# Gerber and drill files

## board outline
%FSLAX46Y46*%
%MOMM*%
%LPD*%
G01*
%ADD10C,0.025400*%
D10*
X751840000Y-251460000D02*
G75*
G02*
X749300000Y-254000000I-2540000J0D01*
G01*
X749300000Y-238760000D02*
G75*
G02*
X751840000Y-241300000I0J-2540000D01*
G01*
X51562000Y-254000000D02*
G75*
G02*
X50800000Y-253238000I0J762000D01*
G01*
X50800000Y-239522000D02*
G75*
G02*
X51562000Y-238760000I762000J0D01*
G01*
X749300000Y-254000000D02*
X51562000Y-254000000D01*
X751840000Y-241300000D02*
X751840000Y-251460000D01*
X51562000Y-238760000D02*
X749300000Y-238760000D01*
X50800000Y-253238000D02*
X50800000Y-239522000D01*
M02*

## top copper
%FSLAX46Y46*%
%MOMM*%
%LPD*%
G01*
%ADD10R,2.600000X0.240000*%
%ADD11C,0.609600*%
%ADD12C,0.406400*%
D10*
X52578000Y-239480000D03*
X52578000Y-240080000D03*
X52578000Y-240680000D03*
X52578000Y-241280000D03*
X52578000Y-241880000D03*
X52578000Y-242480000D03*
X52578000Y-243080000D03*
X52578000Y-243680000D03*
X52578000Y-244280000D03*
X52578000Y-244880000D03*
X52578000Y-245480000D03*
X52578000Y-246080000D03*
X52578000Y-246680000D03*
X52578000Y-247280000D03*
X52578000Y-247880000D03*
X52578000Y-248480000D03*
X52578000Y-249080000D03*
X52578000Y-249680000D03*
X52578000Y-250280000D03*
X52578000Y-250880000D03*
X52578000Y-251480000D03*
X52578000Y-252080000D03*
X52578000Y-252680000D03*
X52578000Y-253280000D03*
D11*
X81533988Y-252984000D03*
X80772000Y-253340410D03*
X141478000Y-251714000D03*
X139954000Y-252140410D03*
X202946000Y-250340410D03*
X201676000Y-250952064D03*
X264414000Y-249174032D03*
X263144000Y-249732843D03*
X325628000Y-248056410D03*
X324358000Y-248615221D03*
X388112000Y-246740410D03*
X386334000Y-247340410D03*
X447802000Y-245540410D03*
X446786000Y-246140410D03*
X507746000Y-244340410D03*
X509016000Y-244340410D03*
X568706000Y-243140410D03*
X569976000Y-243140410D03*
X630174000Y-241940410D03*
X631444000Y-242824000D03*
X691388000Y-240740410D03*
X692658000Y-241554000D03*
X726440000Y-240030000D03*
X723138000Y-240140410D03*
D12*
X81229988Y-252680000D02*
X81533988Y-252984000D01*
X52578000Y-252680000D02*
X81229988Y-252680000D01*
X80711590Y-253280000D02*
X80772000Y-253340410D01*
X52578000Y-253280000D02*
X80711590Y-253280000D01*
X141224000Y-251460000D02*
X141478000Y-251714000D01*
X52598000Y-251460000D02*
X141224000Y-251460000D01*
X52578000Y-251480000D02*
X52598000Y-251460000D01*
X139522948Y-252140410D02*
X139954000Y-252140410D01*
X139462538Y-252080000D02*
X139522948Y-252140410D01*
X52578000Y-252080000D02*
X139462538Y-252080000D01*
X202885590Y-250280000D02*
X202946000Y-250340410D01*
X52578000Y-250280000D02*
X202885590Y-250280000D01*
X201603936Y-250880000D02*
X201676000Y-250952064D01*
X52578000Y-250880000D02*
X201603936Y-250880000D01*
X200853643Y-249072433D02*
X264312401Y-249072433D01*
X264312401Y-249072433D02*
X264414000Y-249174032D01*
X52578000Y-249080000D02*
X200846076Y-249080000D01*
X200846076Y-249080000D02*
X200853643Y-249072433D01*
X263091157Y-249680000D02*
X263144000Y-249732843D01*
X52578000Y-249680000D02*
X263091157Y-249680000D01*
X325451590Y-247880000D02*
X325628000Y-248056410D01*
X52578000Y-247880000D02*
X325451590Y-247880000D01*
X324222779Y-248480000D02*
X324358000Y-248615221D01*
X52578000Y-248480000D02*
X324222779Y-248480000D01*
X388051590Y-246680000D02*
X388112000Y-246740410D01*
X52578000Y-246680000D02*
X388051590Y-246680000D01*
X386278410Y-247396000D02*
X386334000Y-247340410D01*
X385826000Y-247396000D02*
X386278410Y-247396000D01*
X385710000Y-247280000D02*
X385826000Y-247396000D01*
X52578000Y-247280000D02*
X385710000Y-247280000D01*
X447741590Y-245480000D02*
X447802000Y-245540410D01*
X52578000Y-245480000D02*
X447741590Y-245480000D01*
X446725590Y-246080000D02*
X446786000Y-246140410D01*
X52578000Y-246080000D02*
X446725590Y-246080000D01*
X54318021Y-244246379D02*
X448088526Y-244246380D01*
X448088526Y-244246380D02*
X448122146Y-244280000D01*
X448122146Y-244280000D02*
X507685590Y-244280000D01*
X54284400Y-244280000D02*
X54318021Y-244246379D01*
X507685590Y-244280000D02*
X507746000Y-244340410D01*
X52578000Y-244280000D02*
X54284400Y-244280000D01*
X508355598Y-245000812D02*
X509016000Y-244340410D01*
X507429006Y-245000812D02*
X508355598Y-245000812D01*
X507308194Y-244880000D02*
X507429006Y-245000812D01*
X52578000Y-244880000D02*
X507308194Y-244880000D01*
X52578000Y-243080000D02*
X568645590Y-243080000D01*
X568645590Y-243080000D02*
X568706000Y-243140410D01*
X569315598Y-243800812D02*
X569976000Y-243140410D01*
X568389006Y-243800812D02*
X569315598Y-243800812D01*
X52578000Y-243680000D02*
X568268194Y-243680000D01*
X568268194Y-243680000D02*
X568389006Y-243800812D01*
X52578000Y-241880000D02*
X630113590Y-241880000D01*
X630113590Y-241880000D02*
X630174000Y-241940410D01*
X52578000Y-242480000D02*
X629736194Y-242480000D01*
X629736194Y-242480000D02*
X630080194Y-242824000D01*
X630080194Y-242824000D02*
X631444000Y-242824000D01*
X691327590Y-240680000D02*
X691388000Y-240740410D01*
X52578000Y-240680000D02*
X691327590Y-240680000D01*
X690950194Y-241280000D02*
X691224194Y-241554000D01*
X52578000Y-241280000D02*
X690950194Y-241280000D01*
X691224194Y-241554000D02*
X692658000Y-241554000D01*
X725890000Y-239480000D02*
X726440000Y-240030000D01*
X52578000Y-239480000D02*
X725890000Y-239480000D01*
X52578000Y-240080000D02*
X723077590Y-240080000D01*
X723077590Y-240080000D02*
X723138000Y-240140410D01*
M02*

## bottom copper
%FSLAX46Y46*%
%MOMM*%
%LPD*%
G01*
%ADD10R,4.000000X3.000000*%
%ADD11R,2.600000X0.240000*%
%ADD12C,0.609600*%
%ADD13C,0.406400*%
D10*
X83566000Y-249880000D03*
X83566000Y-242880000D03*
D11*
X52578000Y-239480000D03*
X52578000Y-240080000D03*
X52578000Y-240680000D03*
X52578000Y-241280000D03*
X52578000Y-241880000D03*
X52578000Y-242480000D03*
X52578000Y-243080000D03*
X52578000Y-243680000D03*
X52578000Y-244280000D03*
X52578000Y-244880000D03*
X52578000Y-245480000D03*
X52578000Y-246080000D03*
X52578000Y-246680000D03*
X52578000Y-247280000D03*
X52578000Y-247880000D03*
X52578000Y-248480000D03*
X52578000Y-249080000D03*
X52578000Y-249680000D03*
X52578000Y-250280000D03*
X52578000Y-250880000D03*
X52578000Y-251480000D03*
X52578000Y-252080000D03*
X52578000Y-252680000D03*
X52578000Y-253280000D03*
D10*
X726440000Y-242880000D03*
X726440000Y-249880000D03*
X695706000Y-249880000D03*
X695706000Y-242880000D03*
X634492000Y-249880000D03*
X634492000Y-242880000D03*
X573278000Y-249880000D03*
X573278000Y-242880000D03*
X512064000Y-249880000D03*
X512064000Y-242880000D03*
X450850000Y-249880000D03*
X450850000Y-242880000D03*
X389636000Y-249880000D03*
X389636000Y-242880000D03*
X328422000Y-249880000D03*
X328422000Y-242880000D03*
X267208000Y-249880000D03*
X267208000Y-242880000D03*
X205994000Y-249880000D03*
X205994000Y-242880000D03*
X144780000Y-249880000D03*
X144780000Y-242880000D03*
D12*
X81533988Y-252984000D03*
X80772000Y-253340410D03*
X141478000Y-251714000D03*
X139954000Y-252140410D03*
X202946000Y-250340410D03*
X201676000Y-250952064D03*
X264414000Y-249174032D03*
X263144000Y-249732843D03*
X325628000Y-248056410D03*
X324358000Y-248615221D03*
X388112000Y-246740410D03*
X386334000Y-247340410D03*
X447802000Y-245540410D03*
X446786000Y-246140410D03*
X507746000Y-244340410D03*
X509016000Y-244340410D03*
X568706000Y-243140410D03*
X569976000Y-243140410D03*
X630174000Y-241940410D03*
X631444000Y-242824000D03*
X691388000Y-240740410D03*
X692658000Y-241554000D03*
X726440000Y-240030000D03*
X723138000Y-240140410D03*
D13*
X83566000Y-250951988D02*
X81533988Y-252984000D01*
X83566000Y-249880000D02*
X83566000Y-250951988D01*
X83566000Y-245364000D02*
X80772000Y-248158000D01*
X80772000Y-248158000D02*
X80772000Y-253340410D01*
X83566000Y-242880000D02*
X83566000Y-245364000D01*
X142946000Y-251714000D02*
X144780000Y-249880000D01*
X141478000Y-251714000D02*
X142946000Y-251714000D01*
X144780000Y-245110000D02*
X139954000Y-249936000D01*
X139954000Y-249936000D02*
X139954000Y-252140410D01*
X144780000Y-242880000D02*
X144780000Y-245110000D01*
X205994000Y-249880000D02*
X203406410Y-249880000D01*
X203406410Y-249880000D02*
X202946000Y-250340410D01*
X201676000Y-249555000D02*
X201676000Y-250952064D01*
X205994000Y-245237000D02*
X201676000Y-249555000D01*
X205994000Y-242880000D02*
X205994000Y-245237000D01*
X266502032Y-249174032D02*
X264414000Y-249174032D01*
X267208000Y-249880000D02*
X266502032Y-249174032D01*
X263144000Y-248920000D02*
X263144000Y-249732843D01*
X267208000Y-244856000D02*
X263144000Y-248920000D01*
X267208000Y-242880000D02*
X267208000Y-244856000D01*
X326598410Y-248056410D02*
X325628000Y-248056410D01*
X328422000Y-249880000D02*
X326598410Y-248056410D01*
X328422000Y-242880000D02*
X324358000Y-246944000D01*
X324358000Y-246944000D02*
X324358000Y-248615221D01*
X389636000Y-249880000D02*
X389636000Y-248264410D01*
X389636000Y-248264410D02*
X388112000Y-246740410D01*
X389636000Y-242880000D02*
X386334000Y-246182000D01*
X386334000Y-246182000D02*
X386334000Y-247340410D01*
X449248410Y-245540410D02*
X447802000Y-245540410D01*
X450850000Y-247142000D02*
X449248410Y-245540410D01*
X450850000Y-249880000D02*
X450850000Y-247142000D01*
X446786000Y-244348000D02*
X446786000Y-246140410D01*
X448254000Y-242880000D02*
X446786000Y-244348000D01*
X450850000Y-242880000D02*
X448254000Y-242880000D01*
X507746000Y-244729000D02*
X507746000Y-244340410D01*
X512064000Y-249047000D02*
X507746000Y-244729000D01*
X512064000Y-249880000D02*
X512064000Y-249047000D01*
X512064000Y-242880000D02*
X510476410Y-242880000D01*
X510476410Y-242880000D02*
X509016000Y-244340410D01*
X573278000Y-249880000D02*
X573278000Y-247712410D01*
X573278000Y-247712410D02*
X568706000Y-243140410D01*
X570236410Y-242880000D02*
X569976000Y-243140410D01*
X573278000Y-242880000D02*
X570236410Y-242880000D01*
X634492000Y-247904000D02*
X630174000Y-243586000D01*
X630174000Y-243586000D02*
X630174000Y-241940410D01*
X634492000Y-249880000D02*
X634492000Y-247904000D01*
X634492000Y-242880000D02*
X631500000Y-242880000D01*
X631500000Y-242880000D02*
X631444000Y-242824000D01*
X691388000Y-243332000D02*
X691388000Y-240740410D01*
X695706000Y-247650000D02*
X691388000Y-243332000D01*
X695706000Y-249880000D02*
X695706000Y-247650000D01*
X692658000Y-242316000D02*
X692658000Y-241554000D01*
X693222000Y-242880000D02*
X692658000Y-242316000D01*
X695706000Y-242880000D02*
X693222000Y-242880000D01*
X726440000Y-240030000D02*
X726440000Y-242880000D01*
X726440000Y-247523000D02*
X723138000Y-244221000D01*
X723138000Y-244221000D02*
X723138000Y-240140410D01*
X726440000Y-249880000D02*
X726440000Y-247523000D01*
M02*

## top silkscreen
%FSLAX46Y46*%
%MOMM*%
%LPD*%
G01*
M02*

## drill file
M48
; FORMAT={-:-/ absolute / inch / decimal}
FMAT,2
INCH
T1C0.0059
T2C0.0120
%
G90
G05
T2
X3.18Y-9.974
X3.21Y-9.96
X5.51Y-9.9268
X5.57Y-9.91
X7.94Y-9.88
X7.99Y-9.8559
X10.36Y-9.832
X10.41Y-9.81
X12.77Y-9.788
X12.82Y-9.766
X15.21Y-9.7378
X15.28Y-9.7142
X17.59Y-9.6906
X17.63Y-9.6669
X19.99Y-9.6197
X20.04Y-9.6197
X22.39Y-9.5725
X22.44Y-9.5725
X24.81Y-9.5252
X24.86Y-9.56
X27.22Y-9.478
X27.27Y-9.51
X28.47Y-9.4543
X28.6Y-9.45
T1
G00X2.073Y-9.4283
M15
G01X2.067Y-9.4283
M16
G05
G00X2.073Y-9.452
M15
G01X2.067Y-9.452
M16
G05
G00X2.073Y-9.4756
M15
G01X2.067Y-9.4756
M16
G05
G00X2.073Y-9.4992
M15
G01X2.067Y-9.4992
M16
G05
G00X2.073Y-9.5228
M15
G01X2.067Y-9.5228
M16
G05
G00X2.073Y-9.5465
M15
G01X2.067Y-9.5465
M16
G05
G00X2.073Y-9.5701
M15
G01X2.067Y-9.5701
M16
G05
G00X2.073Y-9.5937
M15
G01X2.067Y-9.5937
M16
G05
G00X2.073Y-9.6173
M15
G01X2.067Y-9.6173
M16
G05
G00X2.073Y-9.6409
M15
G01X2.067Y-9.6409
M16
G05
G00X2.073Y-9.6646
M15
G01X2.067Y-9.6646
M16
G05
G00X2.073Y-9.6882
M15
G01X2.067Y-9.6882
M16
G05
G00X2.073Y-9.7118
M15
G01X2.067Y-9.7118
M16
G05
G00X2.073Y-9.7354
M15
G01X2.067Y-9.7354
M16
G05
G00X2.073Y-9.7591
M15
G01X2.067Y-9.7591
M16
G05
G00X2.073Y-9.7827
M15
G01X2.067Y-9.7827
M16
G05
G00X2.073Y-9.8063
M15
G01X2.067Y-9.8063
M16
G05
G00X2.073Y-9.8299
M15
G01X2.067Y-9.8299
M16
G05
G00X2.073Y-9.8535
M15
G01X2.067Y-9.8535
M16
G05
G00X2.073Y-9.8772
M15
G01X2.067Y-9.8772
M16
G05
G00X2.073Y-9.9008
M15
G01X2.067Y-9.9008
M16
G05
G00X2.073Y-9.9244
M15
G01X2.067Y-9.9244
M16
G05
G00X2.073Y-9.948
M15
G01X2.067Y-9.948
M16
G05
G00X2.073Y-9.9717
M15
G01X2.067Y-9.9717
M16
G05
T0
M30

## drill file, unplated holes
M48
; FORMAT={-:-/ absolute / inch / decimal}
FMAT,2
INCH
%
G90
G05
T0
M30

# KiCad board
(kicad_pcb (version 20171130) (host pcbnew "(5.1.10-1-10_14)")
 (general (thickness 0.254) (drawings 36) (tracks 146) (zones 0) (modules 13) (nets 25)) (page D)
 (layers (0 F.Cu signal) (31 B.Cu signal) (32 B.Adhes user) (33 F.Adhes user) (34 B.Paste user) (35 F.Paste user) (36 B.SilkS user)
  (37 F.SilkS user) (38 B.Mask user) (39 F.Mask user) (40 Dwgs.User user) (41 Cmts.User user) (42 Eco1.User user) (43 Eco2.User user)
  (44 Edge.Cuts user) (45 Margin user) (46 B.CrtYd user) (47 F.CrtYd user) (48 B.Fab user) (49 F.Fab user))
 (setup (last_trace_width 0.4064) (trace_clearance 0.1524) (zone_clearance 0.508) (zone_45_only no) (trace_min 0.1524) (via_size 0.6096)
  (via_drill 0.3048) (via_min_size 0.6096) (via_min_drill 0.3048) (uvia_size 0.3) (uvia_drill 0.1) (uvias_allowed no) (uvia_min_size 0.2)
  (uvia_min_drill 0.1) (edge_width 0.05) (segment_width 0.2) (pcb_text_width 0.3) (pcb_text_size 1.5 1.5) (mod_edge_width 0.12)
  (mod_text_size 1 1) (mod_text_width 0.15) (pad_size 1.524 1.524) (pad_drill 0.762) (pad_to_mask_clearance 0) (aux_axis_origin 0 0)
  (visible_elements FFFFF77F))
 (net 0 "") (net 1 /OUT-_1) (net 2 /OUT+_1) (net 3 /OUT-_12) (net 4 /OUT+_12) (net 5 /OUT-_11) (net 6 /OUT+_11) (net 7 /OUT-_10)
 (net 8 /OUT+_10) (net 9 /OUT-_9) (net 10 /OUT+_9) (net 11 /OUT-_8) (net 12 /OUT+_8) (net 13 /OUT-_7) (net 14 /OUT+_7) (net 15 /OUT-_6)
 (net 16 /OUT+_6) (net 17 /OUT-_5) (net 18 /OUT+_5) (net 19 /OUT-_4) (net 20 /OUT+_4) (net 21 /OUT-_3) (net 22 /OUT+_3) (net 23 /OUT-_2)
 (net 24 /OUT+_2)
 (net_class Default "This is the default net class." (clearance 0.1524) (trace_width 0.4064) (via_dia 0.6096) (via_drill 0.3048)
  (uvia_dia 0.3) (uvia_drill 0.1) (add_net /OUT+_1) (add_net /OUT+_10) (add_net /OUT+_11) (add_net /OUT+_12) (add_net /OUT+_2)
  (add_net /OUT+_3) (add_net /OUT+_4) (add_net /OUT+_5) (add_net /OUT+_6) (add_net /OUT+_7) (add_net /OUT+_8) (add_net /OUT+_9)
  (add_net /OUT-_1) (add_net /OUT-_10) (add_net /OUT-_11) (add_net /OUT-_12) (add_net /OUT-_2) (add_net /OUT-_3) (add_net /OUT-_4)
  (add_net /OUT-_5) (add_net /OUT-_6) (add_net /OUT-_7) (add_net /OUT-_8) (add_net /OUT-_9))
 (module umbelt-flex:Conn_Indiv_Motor (layer B.Cu) (at 83.566 246.38 90)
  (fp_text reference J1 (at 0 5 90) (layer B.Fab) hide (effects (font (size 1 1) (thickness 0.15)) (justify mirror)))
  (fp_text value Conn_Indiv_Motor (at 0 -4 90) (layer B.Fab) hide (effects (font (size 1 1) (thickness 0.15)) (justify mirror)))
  (pad 2 smd rect (at -3.5 0 90) (size 3 4) (layers B.Cu B.Mask) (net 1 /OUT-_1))
  (pad 1 smd rect (at 3.5 0 90) (size 3 4) (layers B.Cu B.Mask) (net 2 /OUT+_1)))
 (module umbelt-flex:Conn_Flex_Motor (layer F.Cu) (at 52.578 246.38 180)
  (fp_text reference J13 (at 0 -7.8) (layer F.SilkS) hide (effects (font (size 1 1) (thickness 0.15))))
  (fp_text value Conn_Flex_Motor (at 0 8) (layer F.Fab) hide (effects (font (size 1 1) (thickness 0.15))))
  (pad 24 thru_hole rect (at 0 6.9 180) (size 2.6 0.24) (drill oval 0.3 0.15) (layers *.Cu *.Mask) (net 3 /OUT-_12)
   (solder_paste_margin_ratio -0.2))
  (pad 23 thru_hole rect (at 0 6.3 180) (size 2.6 0.24) (drill oval 0.3 0.15) (layers *.Cu *.Mask) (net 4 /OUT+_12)
   (solder_paste_margin_ratio -0.2))
  (pad 22 thru_hole rect (at 0 5.7 180) (size 2.6 0.24) (drill oval 0.3 0.15) (layers *.Cu *.Mask) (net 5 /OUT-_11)
   (solder_paste_margin_ratio -0.2))
  (pad 21 thru_hole rect (at 0 5.1 180) (size 2.6 0.24) (drill oval 0.3 0.15) (layers *.Cu *.Mask) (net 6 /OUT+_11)
   (solder_paste_margin_ratio -0.2))
  (pad 20 thru_hole rect (at 0 4.5 180) (size 2.6 0.24) (drill oval 0.3 0.15) (layers *.Cu *.Mask) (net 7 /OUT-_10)
   (solder_paste_margin_ratio -0.2))
  (pad 19 thru_hole rect (at 0 3.9 180) (size 2.6 0.24) (drill oval 0.3 0.15) (layers *.Cu *.Mask) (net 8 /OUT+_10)
   (solder_paste_margin_ratio -0.2))
  (pad 18 thru_hole rect (at 0 3.3 180) (size 2.6 0.24) (drill oval 0.3 0.15) (layers *.Cu *.Mask) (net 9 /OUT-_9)
   (solder_paste_margin_ratio -0.2))
  (pad 17 thru_hole rect (at 0 2.7 180) (size 2.6 0.24) (drill oval 0.3 0.15) (layers *.Cu *.Mask) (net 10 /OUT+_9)
   (solder_paste_margin_ratio -0.2))
  (pad 16 thru_hole rect (at 0 2.1 180) (size 2.6 0.24) (drill oval 0.3 0.15) (layers *.Cu *.Mask) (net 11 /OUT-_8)
   (solder_paste_margin_ratio -0.2))
  (pad 15 thru_hole rect (at 0 1.5 180) (size 2.6 0.24) (drill oval 0.3 0.15) (layers *.Cu *.Mask) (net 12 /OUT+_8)
   (solder_paste_margin_ratio -0.2))
  (pad 14 thru_hole rect (at 0 0.9 180) (size 2.6 0.24) (drill oval 0.3 0.15) (layers *.Cu *.Mask) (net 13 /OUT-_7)
   (solder_paste_margin_ratio -0.2))
  (pad 13 thru_hole rect (at 0 0.3 180) (size 2.6 0.24) (drill oval 0.3 0.15) (layers *.Cu *.Mask) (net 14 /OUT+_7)
   (solder_paste_margin_ratio -0.2))
  (pad 12 thru_hole rect (at 0 -0.3 180) (size 2.6 0.24) (drill oval 0.3 0.15) (layers *.Cu *.Mask) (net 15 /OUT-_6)
   (solder_paste_margin_ratio -0.2))
  (pad 11 thru_hole rect (at 0 -0.9 180) (size 2.6 0.24) (drill oval 0.3 0.15) (layers *.Cu *.Mask) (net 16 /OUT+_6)
   (solder_paste_margin_ratio -0.2))
  (pad 10 thru_hole rect (at 0 -1.5 180) (size 2.6 0.24) (drill oval 0.3 0.15) (layers *.Cu *.Mask) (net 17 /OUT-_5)
   (solder_paste_margin_ratio -0.2))
  (pad 9 thru_hole rect (at 0 -2.1 180) (size 2.6 0.24) (drill oval 0.3 0.15) (layers *.Cu *.Mask) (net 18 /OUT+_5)
   (solder_paste_margin_ratio -0.2))
  (pad 8 thru_hole rect (at 0 -2.7 180) (size 2.6 0.24) (drill oval 0.3 0.15) (layers *.Cu *.Mask) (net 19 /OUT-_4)
   (solder_paste_margin_ratio -0.2))
  (pad 7 thru_hole rect (at 0 -3.3 180) (size 2.6 0.24) (drill oval 0.3 0.15) (layers *.Cu *.Mask) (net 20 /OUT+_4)
   (solder_paste_margin_ratio -0.2))
  (pad 6 thru_hole rect (at 0 -3.9 180) (size 2.6 0.24) (drill oval 0.3 0.15) (layers *.Cu *.Mask) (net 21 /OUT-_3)
   (solder_paste_margin_ratio -0.2))
  (pad 5 thru_hole rect (at 0 -4.5 180) (size 2.6 0.24) (drill oval 0.3 0.15) (layers *.Cu *.Mask) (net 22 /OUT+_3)
   (solder_paste_margin_ratio -0.2))
  (pad 4 thru_hole rect (at 0 -5.1 180) (size 2.6 0.24) (drill oval 0.3 0.15) (layers *.Cu *.Mask) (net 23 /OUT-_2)
   (solder_paste_margin_ratio -0.2))
  (pad 3 thru_hole rect (at 0 -5.7 180) (size 2.6 0.24) (drill oval 0.3 0.15) (layers *.Cu *.Mask) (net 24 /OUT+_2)
   (solder_paste_margin_ratio -0.2))
  (pad 2 thru_hole rect (at 0 -6.3 180) (size 2.6 0.24) (drill oval 0.3 0.15) (layers *.Cu *.Mask) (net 1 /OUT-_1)
   (solder_paste_margin_ratio -0.2))
  (pad 1 thru_hole rect (at 0 -6.9 180) (size 2.6 0.24) (drill oval 0.3 0.15) (layers *.Cu *.Mask) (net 2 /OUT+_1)
   (solder_paste_margin_ratio -0.2)))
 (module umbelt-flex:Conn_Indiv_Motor (layer B.Cu) (at 726.44 246.38 270)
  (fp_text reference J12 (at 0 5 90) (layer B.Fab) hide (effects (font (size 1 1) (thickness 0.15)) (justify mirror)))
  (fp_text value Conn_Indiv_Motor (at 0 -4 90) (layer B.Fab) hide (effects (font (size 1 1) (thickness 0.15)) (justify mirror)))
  (pad 2 smd rect (at -3.5 0 270) (size 3 4) (layers B.Cu B.Mask) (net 3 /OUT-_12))
  (pad 1 smd rect (at 3.5 0 270) (size 3 4) (layers B.Cu B.Mask) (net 4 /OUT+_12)))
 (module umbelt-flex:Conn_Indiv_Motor (layer B.Cu) (at 695.706 246.38 90)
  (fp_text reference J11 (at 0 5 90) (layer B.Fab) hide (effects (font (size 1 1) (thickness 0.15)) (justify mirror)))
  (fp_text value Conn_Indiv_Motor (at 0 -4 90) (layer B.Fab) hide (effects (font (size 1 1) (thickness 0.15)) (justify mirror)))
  (pad 2 smd rect (at -3.5 0 90) (size 3 4) (layers B.Cu B.Mask) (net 5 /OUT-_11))
  (pad 1 smd rect (at 3.5 0 90) (size 3 4) (layers B.Cu B.Mask) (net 6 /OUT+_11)))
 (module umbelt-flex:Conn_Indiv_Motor (layer B.Cu) (at 634.492 246.38 90)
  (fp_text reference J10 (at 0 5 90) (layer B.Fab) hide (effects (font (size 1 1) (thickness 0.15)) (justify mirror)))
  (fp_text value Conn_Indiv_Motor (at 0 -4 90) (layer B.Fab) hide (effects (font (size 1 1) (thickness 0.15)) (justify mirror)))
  (pad 2 smd rect (at -3.5 0 90) (size 3 4) (layers B.Cu B.Mask) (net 7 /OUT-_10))
  (pad 1 smd rect (at 3.5 0 90) (size 3 4) (layers B.Cu B.Mask) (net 8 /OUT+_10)))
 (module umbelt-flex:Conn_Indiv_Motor (layer B.Cu) (at 573.278 246.38 90)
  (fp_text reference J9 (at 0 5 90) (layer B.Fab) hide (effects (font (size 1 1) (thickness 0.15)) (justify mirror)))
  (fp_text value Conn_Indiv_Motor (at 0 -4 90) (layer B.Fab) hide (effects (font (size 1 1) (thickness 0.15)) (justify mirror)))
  (pad 2 smd rect (at -3.5 0 90) (size 3 4) (layers B.Cu B.Mask) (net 9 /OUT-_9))
  (pad 1 smd rect (at 3.5 0 90) (size 3 4) (layers B.Cu B.Mask) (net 10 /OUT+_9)))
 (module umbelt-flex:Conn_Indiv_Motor (layer B.Cu) (at 512.064 246.38 90)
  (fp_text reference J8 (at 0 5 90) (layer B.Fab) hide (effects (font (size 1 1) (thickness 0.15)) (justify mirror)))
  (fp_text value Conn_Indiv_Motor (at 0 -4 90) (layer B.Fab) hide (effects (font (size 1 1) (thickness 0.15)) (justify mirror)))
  (pad 2 smd rect (at -3.5 0 90) (size 3 4) (layers B.Cu B.Mask) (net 11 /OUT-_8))
  (pad 1 smd rect (at 3.5 0 90) (size 3 4) (layers B.Cu B.Mask) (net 12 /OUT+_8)))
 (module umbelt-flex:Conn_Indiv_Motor (layer B.Cu) (at 450.85 246.38 90)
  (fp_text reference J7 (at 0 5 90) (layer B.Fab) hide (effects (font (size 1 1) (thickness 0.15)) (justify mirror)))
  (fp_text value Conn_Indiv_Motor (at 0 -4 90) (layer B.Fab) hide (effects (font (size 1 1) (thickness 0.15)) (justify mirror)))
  (pad 2 smd rect (at -3.5 0 90) (size 3 4) (layers B.Cu B.Mask) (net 13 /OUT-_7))
  (pad 1 smd rect (at 3.5 0 90) (size 3 4) (layers B.Cu B.Mask) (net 14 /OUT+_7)))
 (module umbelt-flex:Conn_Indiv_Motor (layer B.Cu) (at 389.636 246.38 90)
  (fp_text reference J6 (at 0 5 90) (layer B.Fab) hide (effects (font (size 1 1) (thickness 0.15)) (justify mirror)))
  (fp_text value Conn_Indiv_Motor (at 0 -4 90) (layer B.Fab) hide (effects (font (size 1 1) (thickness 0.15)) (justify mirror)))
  (pad 2 smd rect (at -3.5 0 90) (size 3 4) (layers B.Cu B.Mask) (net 15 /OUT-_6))
  (pad 1 smd rect (at 3.5 0 90) (size 3 4) (layers B.Cu B.Mask) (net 16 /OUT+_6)))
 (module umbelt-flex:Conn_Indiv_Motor (layer B.Cu) (at 328.422 246.38 90)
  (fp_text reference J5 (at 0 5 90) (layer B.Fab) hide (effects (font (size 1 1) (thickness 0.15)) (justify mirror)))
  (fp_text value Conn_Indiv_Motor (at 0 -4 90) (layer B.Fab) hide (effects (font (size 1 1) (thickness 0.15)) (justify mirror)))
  (pad 2 smd rect (at -3.5 0 90) (size 3 4) (layers B.Cu B.Mask) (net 17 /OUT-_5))
  (pad 1 smd rect (at 3.5 0 90) (size 3 4) (layers B.Cu B.Mask) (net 18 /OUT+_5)))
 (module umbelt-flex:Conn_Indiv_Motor (layer B.Cu) (at 267.208 246.38 90)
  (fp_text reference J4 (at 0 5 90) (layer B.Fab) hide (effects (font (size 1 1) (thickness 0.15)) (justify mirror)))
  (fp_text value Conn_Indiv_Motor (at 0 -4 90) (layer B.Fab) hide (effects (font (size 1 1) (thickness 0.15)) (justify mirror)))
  (pad 2 smd rect (at -3.5 0 90) (size 3 4) (layers B.Cu B.Mask) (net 19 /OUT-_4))
  (pad 1 smd rect (at 3.5 0 90) (size 3 4) (layers B.Cu B.Mask) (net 20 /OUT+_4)))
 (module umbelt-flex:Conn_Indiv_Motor (layer B.Cu) (at 205.994 246.38 90)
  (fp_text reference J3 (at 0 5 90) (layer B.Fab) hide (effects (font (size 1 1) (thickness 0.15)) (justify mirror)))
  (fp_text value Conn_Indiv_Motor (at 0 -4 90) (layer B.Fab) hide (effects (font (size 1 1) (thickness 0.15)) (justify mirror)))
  (pad 2 smd rect (at -3.5 0 90) (size 3 4) (layers B.Cu B.Mask) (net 21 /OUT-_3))
  (pad 1 smd rect (at 3.5 0 90) (size 3 4) (layers B.Cu B.Mask) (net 22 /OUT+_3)))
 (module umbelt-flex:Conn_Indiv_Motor (layer B.Cu) (at 144.78 246.38 90)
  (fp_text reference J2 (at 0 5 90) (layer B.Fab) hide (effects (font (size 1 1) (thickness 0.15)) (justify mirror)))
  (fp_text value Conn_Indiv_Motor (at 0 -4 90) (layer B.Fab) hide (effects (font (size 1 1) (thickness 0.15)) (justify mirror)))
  (pad 2 smd rect (at -3.5 0 90) (size 3 4) (layers B.Cu B.Mask) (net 23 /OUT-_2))
  (pad 1 smd rect (at 3.5 0 90) (size 3 4) (layers B.Cu B.Mask) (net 24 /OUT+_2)))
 (gr_arc (start 749.3 251.46) (end 749.3 254) (angle -90) (layer Edge.Cuts) (width 0.0254))
 (gr_arc (start 749.3 241.3) (end 751.84 241.3) (angle -90) (layer Edge.Cuts) (width 0.0254))
 (gr_arc (start 51.562 253.238) (end 50.8 253.238) (angle -90) (layer Edge.Cuts) (width 0.0254))
 (gr_arc (start 51.562 239.522) (end 51.562 238.76) (angle -90) (layer Edge.Cuts) (width 0.0254))
 (gr_line (start 749.3 254) (end 51.562 254) (layer Edge.Cuts) (width 0.0254))
 (gr_line (start 751.84 241.3) (end 751.84 251.46) (layer Edge.Cuts) (width 0.0254))
 (gr_line (start 51.562 238.76) (end 749.3 238.76) (layer Edge.Cuts) (width 0.0254))
 (gr_line (start 50.8 253.238) (end 50.8 239.522) (layer Edge.Cuts) (width 0.0254))
 (segment (start 83.566 250.951988) (end 81.533988 252.984) (width 0.4064) (layer B.Cu) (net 1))
 (via (at 81.533988 252.984) (size 0.6096) (drill 0.3048) (layers F.Cu B.Cu) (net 1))
 (segment (start 83.566 249.88) (end 83.566 250.951988) (width 0.4064) (layer B.Cu) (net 1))
 (segment (start 81.229988 252.68) (end 81.533988 252.984) (width 0.4064) (layer F.Cu) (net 1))
 (segment (start 52.578 252.68) (end 81.229988 252.68) (width 0.4064) (layer F.Cu) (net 1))
 (via (at 80.772 253.34041) (size 0.6096) (drill 0.3048) (layers F.Cu B.Cu) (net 2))
 (segment (start 80.71159 253.28) (end 80.772 253.34041) (width 0.4064) (layer F.Cu) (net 2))
 (segment (start 52.578 253.28) (end 80.71159 253.28) (width 0.4064) (layer F.Cu) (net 2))
 (segment (start 83.566 245.364) (end 80.772 248.158) (width 0.4064) (layer B.Cu) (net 2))
 (segment (start 80.772 248.158) (end 80.772 253.34041) (width 0.4064) (layer B.Cu) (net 2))
 (segment (start 83.566 242.88) (end 83.566 245.364) (width 0.4064) (layer B.Cu) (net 2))
 (via (at 141.478 251.714) (size 0.6096) (drill 0.3048) (layers F.Cu B.Cu) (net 23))
 (segment (start 142.946 251.714) (end 144.78 249.88) (width 0.4064) (layer B.Cu) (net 23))
 (segment (start 141.478 251.714) (end 142.946 251.714) (width 0.4064) (layer B.Cu) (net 23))
 (segment (start 141.224 251.46) (end 141.478 251.714) (width 0.4064) (layer F.Cu) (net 23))
 (segment (start 52.598 251.46) (end 141.224 251.46) (width 0.4064) (layer F.Cu) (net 23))
 (segment (start 52.578 251.48) (end 52.598 251.46) (width 0.4064) (layer F.Cu) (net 23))
 (via (at 139.954 252.14041) (size 0.6096) (drill 0.3048) (layers F.Cu B.Cu) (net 24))
 (segment (start 139.522948 252.14041) (end 139.954 252.14041) (width 0.4064) (layer F.Cu) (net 24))
 (segment (start 139.462538 252.08) (end 139.522948 252.14041) (width 0.4064) (layer F.Cu) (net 24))
 (segment (start 52.578 252.08) (end 139.462538 252.08) (width 0.4064) (layer F.Cu) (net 24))
 (segment (start 144.78 245.11) (end 139.954 249.936) (width 0.4064) (layer B.Cu) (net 24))
 (segment (start 139.954 249.936) (end 139.954 252.14041) (width 0.4064) (layer B.Cu) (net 24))
 (segment (start 144.78 242.88) (end 144.78 245.11) (width 0.4064) (layer B.Cu) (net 24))
 (segment (start 202.88559 250.28) (end 202.946 250.34041) (width 0.4064) (layer F.Cu) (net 21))
 (via (at 202.946 250.34041) (size 0.6096) (drill 0.3048) (layers F.Cu B.Cu) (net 21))
 (segment (start 52.578 250.28) (end 202.88559 250.28) (width 0.4064) (layer F.Cu) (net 21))
 (segment (start 205.994 249.88) (end 203.40641 249.88) (width 0.4064) (layer B.Cu) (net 21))
 (segment (start 203.40641 249.88) (end 202.946 250.34041) (width 0.4064) (layer B.Cu) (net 21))
 (via (at 201.676 250.952064) (size 0.6096) (drill 0.3048) (layers F.Cu B.Cu) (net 22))
 (segment (start 201.603936 250.88) (end 201.676 250.952064) (width 0.4064) (layer F.Cu) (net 22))
 (segment (start 52.578 250.88) (end 201.603936 250.88) (width 0.4064) (layer F.Cu) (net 22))
 (segment (start 201.676 249.555) (end 201.676 250.952064) (width 0.4064) (layer B.Cu) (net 22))
 (segment (start 205.994 245.237) (end 201.676 249.555) (width 0.4064) (layer B.Cu) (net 22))
 (segment (start 205.994 242.88) (end 205.994 245.237) (width 0.4064) (layer B.Cu) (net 22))
 (segment (start 266.502032 249.174032) (end 264.414 249.174032) (width 0.4064) (layer B.Cu) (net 19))
 (via (at 264.414 249.174032) (size 0.6096) (drill 0.3048) (layers F.Cu B.Cu) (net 19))
 (segment (start 200.853643 249.072433) (end 264.312401 249.072433) (width 0.4064) (layer F.Cu) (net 19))
 (segment (start 264.312401 249.072433) (end 264.414 249.174032) (width 0.4064) (layer F.Cu) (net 19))
 (segment (start 52.578 249.08) (end 200.846076 249.08) (width 0.4064) (layer F.Cu) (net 19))
 (segment (start 200.846076 249.08) (end 200.853643 249.072433) (width 0.4064) (layer F.Cu) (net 19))
 (segment (start 267.208 249.88) (end 266.502032 249.174032) (width 0.4064) (layer B.Cu) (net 19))
 (via (at 263.144 249.732843) (size 0.6096) (drill 0.3048) (layers F.Cu B.Cu) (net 20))
 (segment (start 263.091157 249.68) (end 263.144 249.732843) (width 0.4064) (layer F.Cu) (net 20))
 (segment (start 52.578 249.68) (end 263.091157 249.68) (width 0.4064) (layer F.Cu) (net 20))
 (segment (start 263.144 248.92) (end 263.144 249.732843) (width 0.4064) (layer B.Cu) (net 20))
 (segment (start 267.208 244.856) (end 263.144 248.92) (width 0.4064) (layer B.Cu) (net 20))
 (segment (start 267.208 242.88) (end 267.208 244.856) (width 0.4064) (layer B.Cu) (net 20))
 (via (at 325.628 248.05641) (size 0.6096) (drill 0.3048) (layers F.Cu B.Cu) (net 17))
 (segment (start 326.59841 248.05641) (end 325.628 248.05641) (width 0.4064) (layer B.Cu) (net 17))
 (segment (start 328.422 249.88) (end 326.59841 248.05641) (width 0.4064) (layer B.Cu) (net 17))
 (segment (start 325.45159 247.88) (end 325.628 248.05641) (width 0.4064) (layer F.Cu) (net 17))
 (segment (start 52.578 247.88) (end 325.45159 247.88) (width 0.4064) (layer F.Cu) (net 17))
 (segment (start 328.422 242.88) (end 324.358 246.944) (width 0.4064) (layer B.Cu) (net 18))
 (via (at 324.358 248.615221) (size 0.6096) (drill 0.3048) (layers F.Cu B.Cu) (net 18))
 (segment (start 324.358 246.944) (end 324.358 248.615221) (width 0.4064) (layer B.Cu) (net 18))
 (segment (start 324.222779 248.48) (end 324.358 248.615221) (width 0.4064) (layer F.Cu) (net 18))
 (segment (start 52.578 248.48) (end 324.222779 248.48) (width 0.4064) (layer F.Cu) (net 18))
 (via (at 388.112 246.74041) (size 0.6096) (drill 0.3048) (layers F.Cu B.Cu) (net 15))
 (segment (start 389.636 249.88) (end 389.636 248.26441) (width 0.4064) (layer B.Cu) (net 15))
 (segment (start 389.636 248.26441) (end 388.112 246.74041) (width 0.4064) (layer B.Cu) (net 15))
 (segment (start 388.05159 246.68) (end 388.112 246.74041) (width 0.4064) (layer F.Cu) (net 15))
 (segment (start 52.578 246.68) (end 388.05159 246.68) (width 0.4064) (layer F.Cu) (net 15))
 (via (at 386.334 247.34041) (size 0.6096) (drill 0.3048) (layers F.Cu B.Cu) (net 16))
 (segment (start 389.636 242.88) (end 386.334 246.182) (width 0.4064) (layer B.Cu) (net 16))
 (segment (start 386.334 246.182) (end 386.334 247.34041) (width 0.4064) (layer B.Cu) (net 16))
 (segment (start 386.27841 247.396) (end 386.334 247.34041) (width 0.4064) (layer F.Cu) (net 16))
 (segment (start 385.826 247.396) (end 386.27841 247.396) (width 0.4064) (layer F.Cu) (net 16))
 (segment (start 385.71 247.28) (end 385.826 247.396) (width 0.4064) (layer F.Cu) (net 16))
 (segment (start 52.578 247.28) (end 385.71 247.28) (width 0.4064) (layer F.Cu) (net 16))
 (via (at 447.802 245.54041) (size 0.6096) (drill 0.3048) (layers F.Cu B.Cu) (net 13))
 (segment (start 447.74159 245.48) (end 447.802 245.54041) (width 0.4064) (layer F.Cu) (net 13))
 (segment (start 52.578 245.48) (end 447.74159 245.48) (width 0.4064) (layer F.Cu) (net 13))
 (segment (start 449.24841 245.54041) (end 447.802 245.54041) (width 0.4064) (layer B.Cu) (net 13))
 (segment (start 450.85 247.142) (end 449.24841 245.54041) (width 0.4064) (layer B.Cu) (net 13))
 (segment (start 450.85 249.88) (end 450.85 247.142) (width 0.4064) (layer B.Cu) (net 13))
 (via (at 446.786 246.14041) (size 0.6096) (drill 0.3048) (layers F.Cu B.Cu) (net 14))
 (segment (start 446.72559 246.08) (end 446.786 246.14041) (width 0.4064) (layer F.Cu) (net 14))
 (segment (start 52.578 246.08) (end 446.72559 246.08) (width 0.4064) (layer F.Cu) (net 14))
 (segment (start 446.786 244.348) (end 446.786 246.14041) (width 0.4064) (layer B.Cu) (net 14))
 (segment (start 448.254 242.88) (end 446.786 244.348) (width 0.4064) (layer B.Cu) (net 14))
 (segment (start 450.85 242.88) (end 448.254 242.88) (width 0.4064) (layer B.Cu) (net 14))
 (via (at 507.746 244.34041) (size 0.6096) (drill 0.3048) (layers F.Cu B.Cu) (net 11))
 (segment (start 54.318021 244.246379) (end 448.088526 244.24638) (width 0.4064) (layer F.Cu) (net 11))
 (segment (start 448.088526 244.24638) (end 448.122146 244.28) (width 0.4064) (layer F.Cu) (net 11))
 (segment (start 448.122146 244.28) (end 507.68559 244.28) (width 0.4064) (layer F.Cu) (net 11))
 (segment (start 54.2844 244.28) (end 54.318021 244.246379) (width 0.4064) (layer F.Cu) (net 11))
 (segment (start 507.68559 244.28) (end 507.746 244.34041) (width 0.4064) (layer F.Cu) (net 11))
 (segment (start 52.578 244.28) (end 54.2844 244.28) (width 0.4064) (layer F.Cu) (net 11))
 (segment (start 507.746 244.729) (end 507.746 244.34041) (width 0.4064) (layer B.Cu) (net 11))
 (segment (start 512.064 249.047) (end 507.746 244.729) (width 0.4064) (layer B.Cu) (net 11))
 (segment (start 512.064 249.88) (end 512.064 249.047) (width 0.4064) (layer B.Cu) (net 11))
 (via (at 509.016 244.34041) (size 0.6096) (drill 0.3048) (layers F.Cu B.Cu) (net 12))
 (segment (start 512.064 242.88) (end 510.47641 242.88) (width 0.4064) (layer B.Cu) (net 12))
 (segment (start 510.47641 242.88) (end 509.016 244.34041) (width 0.4064) (layer B.Cu) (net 12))
 (segment (start 508.355598 245.000812) (end 509.016 244.34041) (width 0.4064) (layer F.Cu) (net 12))
 (segment (start 507.429006 245.000812) (end 508.355598 245.000812) (width 0.4064) (layer F.Cu) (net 12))
 (segment (start 507.308194 244.88) (end 507.429006 245.000812) (width 0.4064) (layer F.Cu) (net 12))
 (segment (start 52.578 244.88) (end 507.308194 244.88) (width 0.4064) (layer F.Cu) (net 12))
 (via (at 568.706 243.14041) (size 0.6096) (drill 0.3048) (layers F.Cu B.Cu) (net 9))
 (segment (start 573.278 249.88) (end 573.278 247.71241) (width 0.4064) (layer B.Cu) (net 9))
 (segment (start 573.278 247.71241) (end 568.706 243.14041) (width 0.4064) (layer B.Cu) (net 9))
 (segment (start 52.578 243.08) (end 568.64559 243.08) (width 0.4064) (layer F.Cu) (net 9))
 (segment (start 568.64559 243.08) (end 568.706 243.14041) (width 0.4064) (layer F.Cu) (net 9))
 (via (at 569.976 243.14041) (size 0.6096) (drill 0.3048) (layers F.Cu B.Cu) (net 10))
 (segment (start 570.23641 242.88) (end 569.976 243.14041) (width 0.4064) (layer B.Cu) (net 10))
 (segment (start 573.278 242.88) (end 570.23641 242.88) (width 0.4064) (layer B.Cu) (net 10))
 (segment (start 569.315598 243.800812) (end 569.976 243.14041) (width 0.4064) (layer F.Cu) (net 10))
 (segment (start 568.389006 243.800812) (end 569.315598 243.800812) (width 0.4064) (layer F.Cu) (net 10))
 (segment (start 52.578 243.68) (end 568.268194 243.68) (width 0.4064) (layer F.Cu) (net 10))
 (segment (start 568.268194 243.68) (end 568.389006 243.800812) (width 0.4064) (layer F.Cu) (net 10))
 (via (at 630.174 241.94041) (size 0.6096) (drill 0.3048) (layers F.Cu B.Cu) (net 7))
 (segment (start 52.578 241.88) (end 630.11359 241.88) (width 0.4064) (layer F.Cu) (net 7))
 (segment (start 630.11359 241.88) (end 630.174 241.94041) (width 0.4064) (layer F.Cu) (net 7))
 (segment (start 634.492 247.904) (end 630.174 243.586) (width 0.4064) (layer B.Cu) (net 7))
 (segment (start 630.174 243.586) (end 630.174 241.94041) (width 0.4064) (layer B.Cu) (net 7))
 (segment (start 634.492 249.88) (end 634.492 247.904) (width 0.4064) (layer B.Cu) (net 7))
 (via (at 631.444 242.824) (size 0.6096) (drill 0.3048) (layers F.Cu B.Cu) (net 8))
 (segment (start 634.492 242.88) (end 631.5 242.88) (width 0.4064) (layer B.Cu) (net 8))
 (segment (start 631.5 242.88) (end 631.444 242.824) (width 0.4064) (layer B.Cu) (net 8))
 (segment (start 52.578 242.48) (end 629.736194 242.48) (width 0.4064) (layer F.Cu) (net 8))
 (segment (start 629.736194 242.48) (end 630.080194 242.824) (width 0.4064) (layer F.Cu) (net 8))
 (segment (start 630.080194 242.824) (end 631.444 242.824) (width 0.4064) (layer F.Cu) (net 8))
 (via (at 691.388 240.74041) (size 0.6096) (drill 0.3048) (layers F.Cu B.Cu) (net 5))
 (segment (start 691.32759 240.68) (end 691.388 240.74041) (width 0.4064) (layer F.Cu) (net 5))
 (segment (start 52.578 240.68) (end 691.32759 240.68) (width 0.4064) (layer F.Cu) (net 5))
 (segment (start 691.388 243.332) (end 691.388 240.74041) (width 0.4064) (layer B.Cu) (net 5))
 (segment (start 695.706 247.65) (end 691.388 243.332) (width 0.4064) (layer B.Cu) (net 5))
 (segment (start 695.706 249.88) (end 695.706 247.65) (width 0.4064) (layer B.Cu) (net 5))
 (via (at 692.658 241.554) (size 0.6096) (drill 0.3048) (layers F.Cu B.Cu) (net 6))
 (segment (start 692.658 242.316) (end 692.658 241.554) (width 0.4064) (layer B.Cu) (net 6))
 (segment (start 690.950194 241.28) (end 691.224194 241.554) (width 0.4064) (layer F.Cu) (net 6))
 (segment (start 693.222 242.88) (end 692.658 242.316) (width 0.4064) (layer B.Cu) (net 6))
 (segment (start 695.706 242.88) (end 693.222 242.88) (width 0.4064) (layer B.Cu) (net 6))
 (segment (start 52.578 241.28) (end 690.950194 241.28) (width 0.4064) (layer F.Cu) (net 6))
 (segment (start 691.224194 241.554) (end 692.658 241.554) (width 0.4064) (layer F.Cu) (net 6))
 (via (at 726.44 240.03) (size 0.6096) (drill 0.3048) (layers F.Cu B.Cu) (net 3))
 (segment (start 726.44 240.03) (end 726.44 242.88) (width 0.4064) (layer B.Cu) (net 3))
 (segment (start 725.89 239.48) (end 726.44 240.03) (width 0.4064) (layer F.Cu) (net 3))
 (segment (start 52.578 239.48) (end 725.89 239.48) (width 0.4064) (layer F.Cu) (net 3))
 (segment (start 52.578 240.08) (end 723.07759 240.08) (width 0.4064) (layer F.Cu) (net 4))
 (via (at 723.138 240.14041) (size 0.6096) (drill 0.3048) (layers F.Cu B.Cu) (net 4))
 (segment (start 723.07759 240.08) (end 723.138 240.14041) (width 0.4064) (layer F.Cu) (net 4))
 (segment (start 726.44 247.523) (end 723.138 244.221) (width 0.4064) (layer B.Cu) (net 4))
 (segment (start 723.138 244.221) (end 723.138 240.14041) (width 0.4064) (layer B.Cu) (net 4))
 (segment (start 726.44 249.88) (end 726.44 247.523) (width 0.4064) (layer B.Cu) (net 4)))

